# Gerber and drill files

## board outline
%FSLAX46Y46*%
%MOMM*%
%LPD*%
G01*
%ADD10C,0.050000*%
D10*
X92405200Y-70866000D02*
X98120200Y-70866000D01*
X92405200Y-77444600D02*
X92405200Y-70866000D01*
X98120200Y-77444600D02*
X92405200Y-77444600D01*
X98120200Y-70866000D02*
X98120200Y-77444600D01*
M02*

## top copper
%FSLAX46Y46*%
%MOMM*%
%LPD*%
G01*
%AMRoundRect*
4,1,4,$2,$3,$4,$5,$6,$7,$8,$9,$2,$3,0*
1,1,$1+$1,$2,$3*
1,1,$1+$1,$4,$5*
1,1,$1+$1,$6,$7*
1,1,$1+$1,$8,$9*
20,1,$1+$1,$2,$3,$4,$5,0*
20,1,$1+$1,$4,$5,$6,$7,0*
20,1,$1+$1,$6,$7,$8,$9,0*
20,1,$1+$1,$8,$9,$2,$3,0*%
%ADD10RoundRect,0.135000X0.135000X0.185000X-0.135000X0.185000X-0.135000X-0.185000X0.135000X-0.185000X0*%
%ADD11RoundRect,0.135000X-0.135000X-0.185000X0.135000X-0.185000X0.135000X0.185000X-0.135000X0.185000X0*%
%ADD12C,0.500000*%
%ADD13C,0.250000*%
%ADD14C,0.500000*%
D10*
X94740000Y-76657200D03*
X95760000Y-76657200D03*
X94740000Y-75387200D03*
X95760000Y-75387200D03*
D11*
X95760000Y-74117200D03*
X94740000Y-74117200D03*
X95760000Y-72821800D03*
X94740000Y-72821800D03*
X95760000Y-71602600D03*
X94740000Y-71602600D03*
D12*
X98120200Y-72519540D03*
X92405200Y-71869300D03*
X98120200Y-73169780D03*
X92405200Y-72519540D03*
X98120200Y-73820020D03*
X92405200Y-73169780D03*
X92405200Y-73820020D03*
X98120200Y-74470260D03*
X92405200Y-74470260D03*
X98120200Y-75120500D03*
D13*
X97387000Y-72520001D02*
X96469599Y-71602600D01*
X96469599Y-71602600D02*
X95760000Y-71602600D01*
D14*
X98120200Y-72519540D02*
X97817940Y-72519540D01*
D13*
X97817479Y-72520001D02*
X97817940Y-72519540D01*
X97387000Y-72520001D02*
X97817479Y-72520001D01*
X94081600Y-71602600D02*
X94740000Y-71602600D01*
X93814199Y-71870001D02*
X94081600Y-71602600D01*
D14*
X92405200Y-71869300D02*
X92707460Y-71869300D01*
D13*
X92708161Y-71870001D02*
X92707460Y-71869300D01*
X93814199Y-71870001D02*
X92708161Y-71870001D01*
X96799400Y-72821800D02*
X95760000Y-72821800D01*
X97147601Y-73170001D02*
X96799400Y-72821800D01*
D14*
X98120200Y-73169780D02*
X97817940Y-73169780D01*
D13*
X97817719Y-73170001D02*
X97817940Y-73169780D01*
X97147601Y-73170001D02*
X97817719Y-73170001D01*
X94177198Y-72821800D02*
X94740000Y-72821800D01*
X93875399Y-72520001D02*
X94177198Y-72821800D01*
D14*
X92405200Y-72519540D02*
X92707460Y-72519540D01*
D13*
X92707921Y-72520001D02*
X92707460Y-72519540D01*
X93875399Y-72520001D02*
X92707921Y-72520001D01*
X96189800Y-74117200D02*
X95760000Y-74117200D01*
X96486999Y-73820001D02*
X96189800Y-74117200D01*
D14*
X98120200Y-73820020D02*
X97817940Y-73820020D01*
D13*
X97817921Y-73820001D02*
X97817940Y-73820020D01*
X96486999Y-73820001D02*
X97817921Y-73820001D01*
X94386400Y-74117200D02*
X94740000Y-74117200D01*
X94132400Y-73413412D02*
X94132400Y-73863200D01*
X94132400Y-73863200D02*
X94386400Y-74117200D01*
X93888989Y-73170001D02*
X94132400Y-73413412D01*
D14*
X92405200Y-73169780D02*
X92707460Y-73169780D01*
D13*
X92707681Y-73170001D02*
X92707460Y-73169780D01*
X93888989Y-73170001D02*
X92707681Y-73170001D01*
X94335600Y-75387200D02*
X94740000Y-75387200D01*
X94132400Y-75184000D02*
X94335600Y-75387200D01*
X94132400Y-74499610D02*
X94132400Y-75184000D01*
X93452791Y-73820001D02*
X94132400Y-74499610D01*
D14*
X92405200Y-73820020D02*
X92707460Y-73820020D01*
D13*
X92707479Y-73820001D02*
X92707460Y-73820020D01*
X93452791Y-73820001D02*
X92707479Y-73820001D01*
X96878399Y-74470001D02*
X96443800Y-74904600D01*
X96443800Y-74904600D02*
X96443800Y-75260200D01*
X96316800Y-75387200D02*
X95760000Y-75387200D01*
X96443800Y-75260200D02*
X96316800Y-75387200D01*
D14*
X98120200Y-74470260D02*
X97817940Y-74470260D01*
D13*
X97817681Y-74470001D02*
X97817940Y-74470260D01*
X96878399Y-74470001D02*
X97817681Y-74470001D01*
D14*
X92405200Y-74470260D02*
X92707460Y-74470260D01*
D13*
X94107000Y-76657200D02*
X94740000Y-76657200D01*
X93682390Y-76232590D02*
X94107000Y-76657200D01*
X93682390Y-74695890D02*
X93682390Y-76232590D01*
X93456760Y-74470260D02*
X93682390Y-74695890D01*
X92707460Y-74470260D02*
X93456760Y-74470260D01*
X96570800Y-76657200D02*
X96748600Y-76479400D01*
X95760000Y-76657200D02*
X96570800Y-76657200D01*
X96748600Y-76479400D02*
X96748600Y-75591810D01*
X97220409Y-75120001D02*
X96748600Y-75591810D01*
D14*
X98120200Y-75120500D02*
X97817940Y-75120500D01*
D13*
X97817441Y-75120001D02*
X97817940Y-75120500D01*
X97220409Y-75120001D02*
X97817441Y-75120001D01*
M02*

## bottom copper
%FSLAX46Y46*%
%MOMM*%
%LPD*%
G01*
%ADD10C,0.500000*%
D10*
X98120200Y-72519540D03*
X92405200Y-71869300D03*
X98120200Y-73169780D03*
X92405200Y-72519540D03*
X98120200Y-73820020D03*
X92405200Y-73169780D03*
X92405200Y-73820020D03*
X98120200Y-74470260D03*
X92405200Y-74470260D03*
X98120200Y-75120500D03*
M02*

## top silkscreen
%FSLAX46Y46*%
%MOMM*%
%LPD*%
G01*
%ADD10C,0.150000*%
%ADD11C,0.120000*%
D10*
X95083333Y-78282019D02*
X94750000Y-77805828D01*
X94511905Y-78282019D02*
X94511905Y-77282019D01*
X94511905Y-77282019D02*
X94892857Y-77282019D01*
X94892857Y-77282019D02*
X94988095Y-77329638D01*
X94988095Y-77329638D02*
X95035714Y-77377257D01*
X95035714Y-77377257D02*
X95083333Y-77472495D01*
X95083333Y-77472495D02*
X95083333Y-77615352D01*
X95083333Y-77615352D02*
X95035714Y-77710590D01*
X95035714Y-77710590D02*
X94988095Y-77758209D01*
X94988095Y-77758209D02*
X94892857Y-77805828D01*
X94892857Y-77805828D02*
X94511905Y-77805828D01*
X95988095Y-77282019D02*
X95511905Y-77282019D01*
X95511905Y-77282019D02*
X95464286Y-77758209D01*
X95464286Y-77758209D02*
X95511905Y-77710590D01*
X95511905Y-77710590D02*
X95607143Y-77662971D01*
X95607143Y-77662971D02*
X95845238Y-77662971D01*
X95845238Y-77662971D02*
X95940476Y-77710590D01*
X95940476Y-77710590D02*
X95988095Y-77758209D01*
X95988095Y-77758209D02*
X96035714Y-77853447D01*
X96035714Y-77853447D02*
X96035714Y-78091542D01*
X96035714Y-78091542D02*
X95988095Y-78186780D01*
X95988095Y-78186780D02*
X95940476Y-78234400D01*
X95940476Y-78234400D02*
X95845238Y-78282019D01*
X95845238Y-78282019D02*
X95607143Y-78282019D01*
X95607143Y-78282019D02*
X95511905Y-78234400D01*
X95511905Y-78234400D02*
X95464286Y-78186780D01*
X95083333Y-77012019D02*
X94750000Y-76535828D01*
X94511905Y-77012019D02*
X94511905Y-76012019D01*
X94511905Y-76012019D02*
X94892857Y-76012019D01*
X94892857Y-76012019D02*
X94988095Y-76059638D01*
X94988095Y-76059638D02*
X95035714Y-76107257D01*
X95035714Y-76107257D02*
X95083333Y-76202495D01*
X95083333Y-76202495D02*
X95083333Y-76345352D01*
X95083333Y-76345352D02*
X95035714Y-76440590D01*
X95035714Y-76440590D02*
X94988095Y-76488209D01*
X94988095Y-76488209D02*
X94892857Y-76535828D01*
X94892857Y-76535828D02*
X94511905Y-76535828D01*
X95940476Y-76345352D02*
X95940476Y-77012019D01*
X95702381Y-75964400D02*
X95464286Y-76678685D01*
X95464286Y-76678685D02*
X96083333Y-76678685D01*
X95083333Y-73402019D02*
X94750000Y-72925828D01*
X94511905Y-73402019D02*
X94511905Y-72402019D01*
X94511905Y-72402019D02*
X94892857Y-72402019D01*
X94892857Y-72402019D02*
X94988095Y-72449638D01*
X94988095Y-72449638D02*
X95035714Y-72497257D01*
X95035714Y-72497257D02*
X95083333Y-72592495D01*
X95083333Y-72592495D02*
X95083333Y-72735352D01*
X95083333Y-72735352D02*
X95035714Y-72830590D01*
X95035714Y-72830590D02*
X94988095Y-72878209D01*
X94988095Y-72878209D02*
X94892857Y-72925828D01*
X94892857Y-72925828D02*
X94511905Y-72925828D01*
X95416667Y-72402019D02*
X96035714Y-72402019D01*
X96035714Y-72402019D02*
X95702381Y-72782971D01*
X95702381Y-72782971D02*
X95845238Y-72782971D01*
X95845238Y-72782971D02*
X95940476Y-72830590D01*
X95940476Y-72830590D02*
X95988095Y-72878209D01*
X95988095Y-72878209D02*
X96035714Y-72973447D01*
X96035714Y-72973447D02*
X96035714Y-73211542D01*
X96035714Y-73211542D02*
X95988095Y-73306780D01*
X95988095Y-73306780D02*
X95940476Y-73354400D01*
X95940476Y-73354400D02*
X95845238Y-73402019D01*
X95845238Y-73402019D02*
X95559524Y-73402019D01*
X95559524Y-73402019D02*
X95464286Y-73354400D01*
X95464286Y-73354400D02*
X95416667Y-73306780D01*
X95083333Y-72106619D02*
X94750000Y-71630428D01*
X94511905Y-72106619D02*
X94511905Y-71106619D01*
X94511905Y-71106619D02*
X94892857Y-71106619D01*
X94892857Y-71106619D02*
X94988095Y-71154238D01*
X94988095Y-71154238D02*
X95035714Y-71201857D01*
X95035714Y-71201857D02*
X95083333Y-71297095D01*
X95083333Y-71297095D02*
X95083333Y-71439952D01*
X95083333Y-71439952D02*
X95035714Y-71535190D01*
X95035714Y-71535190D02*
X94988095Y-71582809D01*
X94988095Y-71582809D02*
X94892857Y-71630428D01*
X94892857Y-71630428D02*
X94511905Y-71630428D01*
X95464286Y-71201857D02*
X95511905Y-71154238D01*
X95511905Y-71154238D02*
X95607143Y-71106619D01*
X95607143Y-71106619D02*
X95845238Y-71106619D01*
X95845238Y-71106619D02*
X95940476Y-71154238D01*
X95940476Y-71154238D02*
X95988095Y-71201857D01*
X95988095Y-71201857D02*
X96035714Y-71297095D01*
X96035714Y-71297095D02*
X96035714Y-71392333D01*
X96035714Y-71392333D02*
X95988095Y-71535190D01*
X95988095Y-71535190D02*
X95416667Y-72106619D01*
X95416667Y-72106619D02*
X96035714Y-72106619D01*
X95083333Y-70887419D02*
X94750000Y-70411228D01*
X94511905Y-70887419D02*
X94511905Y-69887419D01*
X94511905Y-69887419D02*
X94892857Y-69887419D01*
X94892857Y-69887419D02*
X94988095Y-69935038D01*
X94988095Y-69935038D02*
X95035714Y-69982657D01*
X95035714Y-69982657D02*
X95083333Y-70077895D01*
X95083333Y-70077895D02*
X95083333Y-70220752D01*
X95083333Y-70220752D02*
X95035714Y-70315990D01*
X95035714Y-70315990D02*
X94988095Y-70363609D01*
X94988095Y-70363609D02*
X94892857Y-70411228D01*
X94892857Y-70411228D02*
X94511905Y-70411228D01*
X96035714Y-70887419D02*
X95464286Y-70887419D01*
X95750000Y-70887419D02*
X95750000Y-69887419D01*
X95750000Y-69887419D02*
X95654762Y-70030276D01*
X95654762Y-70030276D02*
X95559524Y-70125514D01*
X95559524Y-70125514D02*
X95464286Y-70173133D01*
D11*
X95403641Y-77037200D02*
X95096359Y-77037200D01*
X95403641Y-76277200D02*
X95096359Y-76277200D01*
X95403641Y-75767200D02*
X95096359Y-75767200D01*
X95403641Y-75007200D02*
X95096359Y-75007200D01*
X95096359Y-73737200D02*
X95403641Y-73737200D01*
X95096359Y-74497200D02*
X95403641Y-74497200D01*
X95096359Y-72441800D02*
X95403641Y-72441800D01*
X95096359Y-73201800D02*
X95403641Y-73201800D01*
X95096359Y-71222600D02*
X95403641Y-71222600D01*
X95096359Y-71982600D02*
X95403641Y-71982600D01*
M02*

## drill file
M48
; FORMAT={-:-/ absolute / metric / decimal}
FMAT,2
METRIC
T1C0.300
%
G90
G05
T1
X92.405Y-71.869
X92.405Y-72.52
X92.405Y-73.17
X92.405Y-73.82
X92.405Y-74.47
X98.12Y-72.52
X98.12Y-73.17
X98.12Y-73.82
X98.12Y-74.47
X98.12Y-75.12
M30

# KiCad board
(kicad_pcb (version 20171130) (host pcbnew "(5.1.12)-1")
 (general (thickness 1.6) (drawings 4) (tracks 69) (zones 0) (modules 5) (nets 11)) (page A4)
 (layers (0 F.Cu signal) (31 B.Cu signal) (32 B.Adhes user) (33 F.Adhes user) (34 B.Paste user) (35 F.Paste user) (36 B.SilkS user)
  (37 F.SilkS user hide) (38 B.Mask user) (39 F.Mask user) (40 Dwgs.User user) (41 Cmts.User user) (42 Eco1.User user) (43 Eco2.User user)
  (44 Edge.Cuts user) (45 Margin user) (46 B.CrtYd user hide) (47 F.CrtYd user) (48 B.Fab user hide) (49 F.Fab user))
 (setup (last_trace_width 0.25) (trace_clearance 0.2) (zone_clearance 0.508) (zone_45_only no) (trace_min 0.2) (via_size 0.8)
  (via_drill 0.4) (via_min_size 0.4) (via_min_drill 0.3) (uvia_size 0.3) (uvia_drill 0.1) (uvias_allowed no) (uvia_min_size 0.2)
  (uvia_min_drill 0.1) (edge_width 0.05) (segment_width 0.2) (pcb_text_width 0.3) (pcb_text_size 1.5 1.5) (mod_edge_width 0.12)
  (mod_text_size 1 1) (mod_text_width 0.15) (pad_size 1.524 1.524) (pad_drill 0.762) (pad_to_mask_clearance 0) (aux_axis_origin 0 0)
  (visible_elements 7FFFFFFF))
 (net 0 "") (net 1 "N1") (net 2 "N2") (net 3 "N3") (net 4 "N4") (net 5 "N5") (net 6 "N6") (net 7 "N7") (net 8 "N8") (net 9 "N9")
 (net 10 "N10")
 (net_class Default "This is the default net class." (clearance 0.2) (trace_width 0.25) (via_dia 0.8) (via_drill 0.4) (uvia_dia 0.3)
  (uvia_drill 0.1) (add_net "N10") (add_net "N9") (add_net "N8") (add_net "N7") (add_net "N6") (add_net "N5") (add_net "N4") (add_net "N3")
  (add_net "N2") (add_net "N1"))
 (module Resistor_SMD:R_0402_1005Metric (layer F.Cu) (at 95.25 76.6572 180)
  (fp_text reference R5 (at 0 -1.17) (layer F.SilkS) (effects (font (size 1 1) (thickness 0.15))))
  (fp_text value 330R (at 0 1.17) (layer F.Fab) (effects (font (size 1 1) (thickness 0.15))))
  (fp_line (start -0.153641 -0.38) (end 0.153641 -0.38) (layer F.SilkS) (width 0.12))
  (fp_line (start -0.153641 0.38) (end 0.153641 0.38) (layer F.SilkS) (width 0.12))
  (pad 2 smd roundrect (at 0.51 0 180) (size 0.54 0.64) (layers F.Cu F.Paste F.Mask) (roundrect_rratio 0.25) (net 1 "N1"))
  (pad 1 smd roundrect (at -0.51 0 180) (size 0.54 0.64) (layers F.Cu F.Paste F.Mask) (roundrect_rratio 0.25) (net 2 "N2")))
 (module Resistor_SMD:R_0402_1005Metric (layer F.Cu) (at 95.25 75.3872 180)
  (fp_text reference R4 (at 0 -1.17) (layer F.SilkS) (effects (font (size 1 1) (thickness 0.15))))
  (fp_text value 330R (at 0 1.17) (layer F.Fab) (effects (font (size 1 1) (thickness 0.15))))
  (fp_line (start -0.153641 -0.38) (end 0.153641 -0.38) (layer F.SilkS) (width 0.12))
  (fp_line (start -0.153641 0.38) (end 0.153641 0.38) (layer F.SilkS) (width 0.12))
  (pad 2 smd roundrect (at 0.51 0 180) (size 0.54 0.64) (layers F.Cu F.Paste F.Mask) (roundrect_rratio 0.25) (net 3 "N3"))
  (pad 1 smd roundrect (at -0.51 0 180) (size 0.54 0.64) (layers F.Cu F.Paste F.Mask) (roundrect_rratio 0.25) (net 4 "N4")))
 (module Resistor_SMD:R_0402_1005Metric (layer F.Cu) (at 95.25 74.1172)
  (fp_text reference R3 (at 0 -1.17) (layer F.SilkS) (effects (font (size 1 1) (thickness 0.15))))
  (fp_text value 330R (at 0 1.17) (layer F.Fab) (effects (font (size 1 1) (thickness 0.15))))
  (fp_line (start -0.153641 -0.38) (end 0.153641 -0.38) (layer F.SilkS) (width 0.12))
  (fp_line (start -0.153641 0.38) (end 0.153641 0.38) (layer F.SilkS) (width 0.12))
  (pad 2 smd roundrect (at 0.51 0) (size 0.54 0.64) (layers F.Cu F.Paste F.Mask) (roundrect_rratio 0.25) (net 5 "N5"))
  (pad 1 smd roundrect (at -0.51 0) (size 0.54 0.64) (layers F.Cu F.Paste F.Mask) (roundrect_rratio 0.25) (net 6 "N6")))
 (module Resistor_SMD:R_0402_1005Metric (layer F.Cu) (at 95.25 72.8218)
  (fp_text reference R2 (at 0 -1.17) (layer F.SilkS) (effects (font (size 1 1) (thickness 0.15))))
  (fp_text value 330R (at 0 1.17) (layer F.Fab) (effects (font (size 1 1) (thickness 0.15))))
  (fp_line (start -0.153641 -0.38) (end 0.153641 -0.38) (layer F.SilkS) (width 0.12))
  (fp_line (start -0.153641 0.38) (end 0.153641 0.38) (layer F.SilkS) (width 0.12))
  (pad 2 smd roundrect (at 0.51 0) (size 0.54 0.64) (layers F.Cu F.Paste F.Mask) (roundrect_rratio 0.25) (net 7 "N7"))
  (pad 1 smd roundrect (at -0.51 0) (size 0.54 0.64) (layers F.Cu F.Paste F.Mask) (roundrect_rratio 0.25) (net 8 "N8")))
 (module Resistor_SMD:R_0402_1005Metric (layer F.Cu) (at 95.25 71.6026)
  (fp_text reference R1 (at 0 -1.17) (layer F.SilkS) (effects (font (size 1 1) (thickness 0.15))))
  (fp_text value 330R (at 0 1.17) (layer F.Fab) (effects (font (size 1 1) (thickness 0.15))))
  (fp_line (start -0.153641 -0.38) (end 0.153641 -0.38) (layer F.SilkS) (width 0.12))
  (fp_line (start -0.153641 0.38) (end 0.153641 0.38) (layer F.SilkS) (width 0.12))
  (pad 2 smd roundrect (at 0.51 0) (size 0.54 0.64) (layers F.Cu F.Paste F.Mask) (roundrect_rratio 0.25) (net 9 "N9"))
  (pad 1 smd roundrect (at -0.51 0) (size 0.54 0.64) (layers F.Cu F.Paste F.Mask) (roundrect_rratio 0.25) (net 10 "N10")))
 (gr_line (start 92.4052 70.866) (end 98.1202 70.866) (layer Edge.Cuts) (width 0.05))
 (gr_line (start 92.4052 77.4446) (end 92.4052 70.866) (layer Edge.Cuts) (width 0.05))
 (gr_line (start 98.1202 77.4446) (end 92.4052 77.4446) (layer Edge.Cuts) (width 0.05))
 (gr_line (start 98.1202 70.866) (end 98.1202 77.4446) (layer Edge.Cuts) (width 0.05))
 (via (at 98.1202 72.51954) (size 0.5) (drill 0.3) (layers F.Cu B.Cu) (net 9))
 (segment (start 97.387 72.520001) (end 96.469599 71.6026) (width 0.25) (layer F.Cu) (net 9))
 (segment (start 96.469599 71.6026) (end 95.76 71.6026) (width 0.25) (layer F.Cu) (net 9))
 (segment (start 98.1202 72.51954) (end 97.81794 72.51954) (width 0.5) (layer F.Cu) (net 9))
 (segment (start 97.817479 72.520001) (end 97.81794 72.51954) (width 0.25) (layer F.Cu) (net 9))
 (segment (start 97.387 72.520001) (end 97.817479 72.520001) (width 0.25) (layer F.Cu) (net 9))
 (via (at 92.4052 71.8693) (size 0.5) (drill 0.3) (layers F.Cu B.Cu) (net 10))
 (segment (start 94.0816 71.6026) (end 94.74 71.6026) (width 0.25) (layer F.Cu) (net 10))
 (segment (start 93.814199 71.870001) (end 94.0816 71.6026) (width 0.25) (layer F.Cu) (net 10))
 (segment (start 92.4052 71.8693) (end 92.70746 71.8693) (width 0.5) (layer F.Cu) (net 10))
 (segment (start 92.708161 71.870001) (end 92.70746 71.8693) (width 0.25) (layer F.Cu) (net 10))
 (segment (start 93.814199 71.870001) (end 92.708161 71.870001) (width 0.25) (layer F.Cu) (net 10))
 (via (at 98.1202 73.16978) (size 0.5) (drill 0.3) (layers F.Cu B.Cu) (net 7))
 (segment (start 96.7994 72.8218) (end 95.76 72.8218) (width 0.25) (layer F.Cu) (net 7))
 (segment (start 97.147601 73.170001) (end 96.7994 72.8218) (width 0.25) (layer F.Cu) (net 7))
 (segment (start 98.1202 73.16978) (end 97.81794 73.16978) (width 0.5) (layer F.Cu) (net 7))
 (segment (start 97.817719 73.170001) (end 97.81794 73.16978) (width 0.25) (layer F.Cu) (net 7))
 (segment (start 97.147601 73.170001) (end 97.817719 73.170001) (width 0.25) (layer F.Cu) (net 7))
 (via (at 92.4052 72.51954) (size 0.5) (drill 0.3) (layers F.Cu B.Cu) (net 8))
 (segment (start 94.177198 72.8218) (end 94.74 72.8218) (width 0.25) (layer F.Cu) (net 8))
 (segment (start 93.875399 72.520001) (end 94.177198 72.8218) (width 0.25) (layer F.Cu) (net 8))
 (segment (start 92.4052 72.51954) (end 92.70746 72.51954) (width 0.5) (layer F.Cu) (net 8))
 (segment (start 92.707921 72.520001) (end 92.70746 72.51954) (width 0.25) (layer F.Cu) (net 8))
 (segment (start 93.875399 72.520001) (end 92.707921 72.520001) (width 0.25) (layer F.Cu) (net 8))
 (via (at 98.1202 73.82002) (size 0.5) (drill 0.3) (layers F.Cu B.Cu) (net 5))
 (segment (start 96.1898 74.1172) (end 95.76 74.1172) (width 0.25) (layer F.Cu) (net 5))
 (segment (start 96.486999 73.820001) (end 96.1898 74.1172) (width 0.25) (layer F.Cu) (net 5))
 (segment (start 98.1202 73.82002) (end 97.81794 73.82002) (width 0.5) (layer F.Cu) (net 5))
 (segment (start 97.817921 73.820001) (end 97.81794 73.82002) (width 0.25) (layer F.Cu) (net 5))
 (segment (start 96.486999 73.820001) (end 97.817921 73.820001) (width 0.25) (layer F.Cu) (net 5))
 (via (at 92.4052 73.16978) (size 0.5) (drill 0.3) (layers F.Cu B.Cu) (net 6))
 (segment (start 94.3864 74.1172) (end 94.74 74.1172) (width 0.25) (layer F.Cu) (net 6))
 (segment (start 94.1324 73.413412) (end 94.1324 73.8632) (width 0.25) (layer F.Cu) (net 6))
 (segment (start 94.1324 73.8632) (end 94.3864 74.1172) (width 0.25) (layer F.Cu) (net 6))
 (segment (start 93.888989 73.170001) (end 94.1324 73.413412) (width 0.25) (layer F.Cu) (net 6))
 (segment (start 92.4052 73.16978) (end 92.70746 73.16978) (width 0.5) (layer F.Cu) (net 6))
 (segment (start 92.707681 73.170001) (end 92.70746 73.16978) (width 0.25) (layer F.Cu) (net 6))
 (segment (start 93.888989 73.170001) (end 92.707681 73.170001) (width 0.25) (layer F.Cu) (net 6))
 (via (at 92.4052 73.82002) (size 0.5) (drill 0.3) (layers F.Cu B.Cu) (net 3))
 (segment (start 94.3356 75.3872) (end 94.74 75.3872) (width 0.25) (layer F.Cu) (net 3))
 (segment (start 94.1324 75.184) (end 94.3356 75.3872) (width 0.25) (layer F.Cu) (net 3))
 (segment (start 94.1324 74.49961) (end 94.1324 75.184) (width 0.25) (layer F.Cu) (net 3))
 (segment (start 93.452791 73.820001) (end 94.1324 74.49961) (width 0.25) (layer F.Cu) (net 3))
 (segment (start 92.4052 73.82002) (end 92.70746 73.82002) (width 0.5) (layer F.Cu) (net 3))
 (segment (start 92.707479 73.820001) (end 92.70746 73.82002) (width 0.25) (layer F.Cu) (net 3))
 (segment (start 93.452791 73.820001) (end 92.707479 73.820001) (width 0.25) (layer F.Cu) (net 3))
 (via (at 98.1202 74.47026) (size 0.5) (drill 0.3) (layers F.Cu B.Cu) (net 4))
 (segment (start 96.878399 74.470001) (end 96.4438 74.9046) (width 0.25) (layer F.Cu) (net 4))
 (segment (start 96.4438 74.9046) (end 96.4438 75.2602) (width 0.25) (layer F.Cu) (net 4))
 (segment (start 96.3168 75.3872) (end 95.76 75.3872) (width 0.25) (layer F.Cu) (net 4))
 (segment (start 96.4438 75.2602) (end 96.3168 75.3872) (width 0.25) (layer F.Cu) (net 4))
 (segment (start 98.1202 74.47026) (end 97.81794 74.47026) (width 0.5) (layer F.Cu) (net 4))
 (segment (start 97.817681 74.470001) (end 97.81794 74.47026) (width 0.25) (layer F.Cu) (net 4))
 (segment (start 96.878399 74.470001) (end 97.817681 74.470001) (width 0.25) (layer F.Cu) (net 4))
 (via (at 92.4052 74.47026) (size 0.5) (drill 0.3) (layers F.Cu B.Cu) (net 1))
 (segment (start 92.4052 74.47026) (end 92.70746 74.47026) (width 0.5) (layer F.Cu) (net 1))
 (segment (start 94.107 76.6572) (end 94.74 76.6572) (width 0.25) (layer F.Cu) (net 1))
 (segment (start 93.68239 76.23259) (end 94.107 76.6572) (width 0.25) (layer F.Cu) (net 1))
 (segment (start 93.68239 74.69589) (end 93.68239 76.23259) (width 0.25) (layer F.Cu) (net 1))
 (segment (start 93.45676 74.47026) (end 93.68239 74.69589) (width 0.25) (layer F.Cu) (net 1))
 (segment (start 92.70746 74.47026) (end 93.45676 74.47026) (width 0.25) (layer F.Cu) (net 1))
 (via (at 98.1202 75.1205) (size 0.5) (drill 0.3) (layers F.Cu B.Cu) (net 2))
 (segment (start 96.5708 76.6572) (end 96.7486 76.4794) (width 0.25) (layer F.Cu) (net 2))
 (segment (start 95.76 76.6572) (end 96.5708 76.6572) (width 0.25) (layer F.Cu) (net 2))
 (segment (start 96.7486 76.4794) (end 96.7486 75.59181) (width 0.25) (layer F.Cu) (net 2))
 (segment (start 97.220409 75.120001) (end 96.7486 75.59181) (width 0.25) (layer F.Cu) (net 2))
 (segment (start 98.1202 75.1205) (end 97.81794 75.1205) (width 0.5) (layer F.Cu) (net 2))
 (segment (start 97.817441 75.120001) (end 97.81794 75.1205) (width 0.25) (layer F.Cu) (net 2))
 (segment (start 97.220409 75.120001) (end 97.817441 75.120001) (width 0.25) (layer F.Cu) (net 2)))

